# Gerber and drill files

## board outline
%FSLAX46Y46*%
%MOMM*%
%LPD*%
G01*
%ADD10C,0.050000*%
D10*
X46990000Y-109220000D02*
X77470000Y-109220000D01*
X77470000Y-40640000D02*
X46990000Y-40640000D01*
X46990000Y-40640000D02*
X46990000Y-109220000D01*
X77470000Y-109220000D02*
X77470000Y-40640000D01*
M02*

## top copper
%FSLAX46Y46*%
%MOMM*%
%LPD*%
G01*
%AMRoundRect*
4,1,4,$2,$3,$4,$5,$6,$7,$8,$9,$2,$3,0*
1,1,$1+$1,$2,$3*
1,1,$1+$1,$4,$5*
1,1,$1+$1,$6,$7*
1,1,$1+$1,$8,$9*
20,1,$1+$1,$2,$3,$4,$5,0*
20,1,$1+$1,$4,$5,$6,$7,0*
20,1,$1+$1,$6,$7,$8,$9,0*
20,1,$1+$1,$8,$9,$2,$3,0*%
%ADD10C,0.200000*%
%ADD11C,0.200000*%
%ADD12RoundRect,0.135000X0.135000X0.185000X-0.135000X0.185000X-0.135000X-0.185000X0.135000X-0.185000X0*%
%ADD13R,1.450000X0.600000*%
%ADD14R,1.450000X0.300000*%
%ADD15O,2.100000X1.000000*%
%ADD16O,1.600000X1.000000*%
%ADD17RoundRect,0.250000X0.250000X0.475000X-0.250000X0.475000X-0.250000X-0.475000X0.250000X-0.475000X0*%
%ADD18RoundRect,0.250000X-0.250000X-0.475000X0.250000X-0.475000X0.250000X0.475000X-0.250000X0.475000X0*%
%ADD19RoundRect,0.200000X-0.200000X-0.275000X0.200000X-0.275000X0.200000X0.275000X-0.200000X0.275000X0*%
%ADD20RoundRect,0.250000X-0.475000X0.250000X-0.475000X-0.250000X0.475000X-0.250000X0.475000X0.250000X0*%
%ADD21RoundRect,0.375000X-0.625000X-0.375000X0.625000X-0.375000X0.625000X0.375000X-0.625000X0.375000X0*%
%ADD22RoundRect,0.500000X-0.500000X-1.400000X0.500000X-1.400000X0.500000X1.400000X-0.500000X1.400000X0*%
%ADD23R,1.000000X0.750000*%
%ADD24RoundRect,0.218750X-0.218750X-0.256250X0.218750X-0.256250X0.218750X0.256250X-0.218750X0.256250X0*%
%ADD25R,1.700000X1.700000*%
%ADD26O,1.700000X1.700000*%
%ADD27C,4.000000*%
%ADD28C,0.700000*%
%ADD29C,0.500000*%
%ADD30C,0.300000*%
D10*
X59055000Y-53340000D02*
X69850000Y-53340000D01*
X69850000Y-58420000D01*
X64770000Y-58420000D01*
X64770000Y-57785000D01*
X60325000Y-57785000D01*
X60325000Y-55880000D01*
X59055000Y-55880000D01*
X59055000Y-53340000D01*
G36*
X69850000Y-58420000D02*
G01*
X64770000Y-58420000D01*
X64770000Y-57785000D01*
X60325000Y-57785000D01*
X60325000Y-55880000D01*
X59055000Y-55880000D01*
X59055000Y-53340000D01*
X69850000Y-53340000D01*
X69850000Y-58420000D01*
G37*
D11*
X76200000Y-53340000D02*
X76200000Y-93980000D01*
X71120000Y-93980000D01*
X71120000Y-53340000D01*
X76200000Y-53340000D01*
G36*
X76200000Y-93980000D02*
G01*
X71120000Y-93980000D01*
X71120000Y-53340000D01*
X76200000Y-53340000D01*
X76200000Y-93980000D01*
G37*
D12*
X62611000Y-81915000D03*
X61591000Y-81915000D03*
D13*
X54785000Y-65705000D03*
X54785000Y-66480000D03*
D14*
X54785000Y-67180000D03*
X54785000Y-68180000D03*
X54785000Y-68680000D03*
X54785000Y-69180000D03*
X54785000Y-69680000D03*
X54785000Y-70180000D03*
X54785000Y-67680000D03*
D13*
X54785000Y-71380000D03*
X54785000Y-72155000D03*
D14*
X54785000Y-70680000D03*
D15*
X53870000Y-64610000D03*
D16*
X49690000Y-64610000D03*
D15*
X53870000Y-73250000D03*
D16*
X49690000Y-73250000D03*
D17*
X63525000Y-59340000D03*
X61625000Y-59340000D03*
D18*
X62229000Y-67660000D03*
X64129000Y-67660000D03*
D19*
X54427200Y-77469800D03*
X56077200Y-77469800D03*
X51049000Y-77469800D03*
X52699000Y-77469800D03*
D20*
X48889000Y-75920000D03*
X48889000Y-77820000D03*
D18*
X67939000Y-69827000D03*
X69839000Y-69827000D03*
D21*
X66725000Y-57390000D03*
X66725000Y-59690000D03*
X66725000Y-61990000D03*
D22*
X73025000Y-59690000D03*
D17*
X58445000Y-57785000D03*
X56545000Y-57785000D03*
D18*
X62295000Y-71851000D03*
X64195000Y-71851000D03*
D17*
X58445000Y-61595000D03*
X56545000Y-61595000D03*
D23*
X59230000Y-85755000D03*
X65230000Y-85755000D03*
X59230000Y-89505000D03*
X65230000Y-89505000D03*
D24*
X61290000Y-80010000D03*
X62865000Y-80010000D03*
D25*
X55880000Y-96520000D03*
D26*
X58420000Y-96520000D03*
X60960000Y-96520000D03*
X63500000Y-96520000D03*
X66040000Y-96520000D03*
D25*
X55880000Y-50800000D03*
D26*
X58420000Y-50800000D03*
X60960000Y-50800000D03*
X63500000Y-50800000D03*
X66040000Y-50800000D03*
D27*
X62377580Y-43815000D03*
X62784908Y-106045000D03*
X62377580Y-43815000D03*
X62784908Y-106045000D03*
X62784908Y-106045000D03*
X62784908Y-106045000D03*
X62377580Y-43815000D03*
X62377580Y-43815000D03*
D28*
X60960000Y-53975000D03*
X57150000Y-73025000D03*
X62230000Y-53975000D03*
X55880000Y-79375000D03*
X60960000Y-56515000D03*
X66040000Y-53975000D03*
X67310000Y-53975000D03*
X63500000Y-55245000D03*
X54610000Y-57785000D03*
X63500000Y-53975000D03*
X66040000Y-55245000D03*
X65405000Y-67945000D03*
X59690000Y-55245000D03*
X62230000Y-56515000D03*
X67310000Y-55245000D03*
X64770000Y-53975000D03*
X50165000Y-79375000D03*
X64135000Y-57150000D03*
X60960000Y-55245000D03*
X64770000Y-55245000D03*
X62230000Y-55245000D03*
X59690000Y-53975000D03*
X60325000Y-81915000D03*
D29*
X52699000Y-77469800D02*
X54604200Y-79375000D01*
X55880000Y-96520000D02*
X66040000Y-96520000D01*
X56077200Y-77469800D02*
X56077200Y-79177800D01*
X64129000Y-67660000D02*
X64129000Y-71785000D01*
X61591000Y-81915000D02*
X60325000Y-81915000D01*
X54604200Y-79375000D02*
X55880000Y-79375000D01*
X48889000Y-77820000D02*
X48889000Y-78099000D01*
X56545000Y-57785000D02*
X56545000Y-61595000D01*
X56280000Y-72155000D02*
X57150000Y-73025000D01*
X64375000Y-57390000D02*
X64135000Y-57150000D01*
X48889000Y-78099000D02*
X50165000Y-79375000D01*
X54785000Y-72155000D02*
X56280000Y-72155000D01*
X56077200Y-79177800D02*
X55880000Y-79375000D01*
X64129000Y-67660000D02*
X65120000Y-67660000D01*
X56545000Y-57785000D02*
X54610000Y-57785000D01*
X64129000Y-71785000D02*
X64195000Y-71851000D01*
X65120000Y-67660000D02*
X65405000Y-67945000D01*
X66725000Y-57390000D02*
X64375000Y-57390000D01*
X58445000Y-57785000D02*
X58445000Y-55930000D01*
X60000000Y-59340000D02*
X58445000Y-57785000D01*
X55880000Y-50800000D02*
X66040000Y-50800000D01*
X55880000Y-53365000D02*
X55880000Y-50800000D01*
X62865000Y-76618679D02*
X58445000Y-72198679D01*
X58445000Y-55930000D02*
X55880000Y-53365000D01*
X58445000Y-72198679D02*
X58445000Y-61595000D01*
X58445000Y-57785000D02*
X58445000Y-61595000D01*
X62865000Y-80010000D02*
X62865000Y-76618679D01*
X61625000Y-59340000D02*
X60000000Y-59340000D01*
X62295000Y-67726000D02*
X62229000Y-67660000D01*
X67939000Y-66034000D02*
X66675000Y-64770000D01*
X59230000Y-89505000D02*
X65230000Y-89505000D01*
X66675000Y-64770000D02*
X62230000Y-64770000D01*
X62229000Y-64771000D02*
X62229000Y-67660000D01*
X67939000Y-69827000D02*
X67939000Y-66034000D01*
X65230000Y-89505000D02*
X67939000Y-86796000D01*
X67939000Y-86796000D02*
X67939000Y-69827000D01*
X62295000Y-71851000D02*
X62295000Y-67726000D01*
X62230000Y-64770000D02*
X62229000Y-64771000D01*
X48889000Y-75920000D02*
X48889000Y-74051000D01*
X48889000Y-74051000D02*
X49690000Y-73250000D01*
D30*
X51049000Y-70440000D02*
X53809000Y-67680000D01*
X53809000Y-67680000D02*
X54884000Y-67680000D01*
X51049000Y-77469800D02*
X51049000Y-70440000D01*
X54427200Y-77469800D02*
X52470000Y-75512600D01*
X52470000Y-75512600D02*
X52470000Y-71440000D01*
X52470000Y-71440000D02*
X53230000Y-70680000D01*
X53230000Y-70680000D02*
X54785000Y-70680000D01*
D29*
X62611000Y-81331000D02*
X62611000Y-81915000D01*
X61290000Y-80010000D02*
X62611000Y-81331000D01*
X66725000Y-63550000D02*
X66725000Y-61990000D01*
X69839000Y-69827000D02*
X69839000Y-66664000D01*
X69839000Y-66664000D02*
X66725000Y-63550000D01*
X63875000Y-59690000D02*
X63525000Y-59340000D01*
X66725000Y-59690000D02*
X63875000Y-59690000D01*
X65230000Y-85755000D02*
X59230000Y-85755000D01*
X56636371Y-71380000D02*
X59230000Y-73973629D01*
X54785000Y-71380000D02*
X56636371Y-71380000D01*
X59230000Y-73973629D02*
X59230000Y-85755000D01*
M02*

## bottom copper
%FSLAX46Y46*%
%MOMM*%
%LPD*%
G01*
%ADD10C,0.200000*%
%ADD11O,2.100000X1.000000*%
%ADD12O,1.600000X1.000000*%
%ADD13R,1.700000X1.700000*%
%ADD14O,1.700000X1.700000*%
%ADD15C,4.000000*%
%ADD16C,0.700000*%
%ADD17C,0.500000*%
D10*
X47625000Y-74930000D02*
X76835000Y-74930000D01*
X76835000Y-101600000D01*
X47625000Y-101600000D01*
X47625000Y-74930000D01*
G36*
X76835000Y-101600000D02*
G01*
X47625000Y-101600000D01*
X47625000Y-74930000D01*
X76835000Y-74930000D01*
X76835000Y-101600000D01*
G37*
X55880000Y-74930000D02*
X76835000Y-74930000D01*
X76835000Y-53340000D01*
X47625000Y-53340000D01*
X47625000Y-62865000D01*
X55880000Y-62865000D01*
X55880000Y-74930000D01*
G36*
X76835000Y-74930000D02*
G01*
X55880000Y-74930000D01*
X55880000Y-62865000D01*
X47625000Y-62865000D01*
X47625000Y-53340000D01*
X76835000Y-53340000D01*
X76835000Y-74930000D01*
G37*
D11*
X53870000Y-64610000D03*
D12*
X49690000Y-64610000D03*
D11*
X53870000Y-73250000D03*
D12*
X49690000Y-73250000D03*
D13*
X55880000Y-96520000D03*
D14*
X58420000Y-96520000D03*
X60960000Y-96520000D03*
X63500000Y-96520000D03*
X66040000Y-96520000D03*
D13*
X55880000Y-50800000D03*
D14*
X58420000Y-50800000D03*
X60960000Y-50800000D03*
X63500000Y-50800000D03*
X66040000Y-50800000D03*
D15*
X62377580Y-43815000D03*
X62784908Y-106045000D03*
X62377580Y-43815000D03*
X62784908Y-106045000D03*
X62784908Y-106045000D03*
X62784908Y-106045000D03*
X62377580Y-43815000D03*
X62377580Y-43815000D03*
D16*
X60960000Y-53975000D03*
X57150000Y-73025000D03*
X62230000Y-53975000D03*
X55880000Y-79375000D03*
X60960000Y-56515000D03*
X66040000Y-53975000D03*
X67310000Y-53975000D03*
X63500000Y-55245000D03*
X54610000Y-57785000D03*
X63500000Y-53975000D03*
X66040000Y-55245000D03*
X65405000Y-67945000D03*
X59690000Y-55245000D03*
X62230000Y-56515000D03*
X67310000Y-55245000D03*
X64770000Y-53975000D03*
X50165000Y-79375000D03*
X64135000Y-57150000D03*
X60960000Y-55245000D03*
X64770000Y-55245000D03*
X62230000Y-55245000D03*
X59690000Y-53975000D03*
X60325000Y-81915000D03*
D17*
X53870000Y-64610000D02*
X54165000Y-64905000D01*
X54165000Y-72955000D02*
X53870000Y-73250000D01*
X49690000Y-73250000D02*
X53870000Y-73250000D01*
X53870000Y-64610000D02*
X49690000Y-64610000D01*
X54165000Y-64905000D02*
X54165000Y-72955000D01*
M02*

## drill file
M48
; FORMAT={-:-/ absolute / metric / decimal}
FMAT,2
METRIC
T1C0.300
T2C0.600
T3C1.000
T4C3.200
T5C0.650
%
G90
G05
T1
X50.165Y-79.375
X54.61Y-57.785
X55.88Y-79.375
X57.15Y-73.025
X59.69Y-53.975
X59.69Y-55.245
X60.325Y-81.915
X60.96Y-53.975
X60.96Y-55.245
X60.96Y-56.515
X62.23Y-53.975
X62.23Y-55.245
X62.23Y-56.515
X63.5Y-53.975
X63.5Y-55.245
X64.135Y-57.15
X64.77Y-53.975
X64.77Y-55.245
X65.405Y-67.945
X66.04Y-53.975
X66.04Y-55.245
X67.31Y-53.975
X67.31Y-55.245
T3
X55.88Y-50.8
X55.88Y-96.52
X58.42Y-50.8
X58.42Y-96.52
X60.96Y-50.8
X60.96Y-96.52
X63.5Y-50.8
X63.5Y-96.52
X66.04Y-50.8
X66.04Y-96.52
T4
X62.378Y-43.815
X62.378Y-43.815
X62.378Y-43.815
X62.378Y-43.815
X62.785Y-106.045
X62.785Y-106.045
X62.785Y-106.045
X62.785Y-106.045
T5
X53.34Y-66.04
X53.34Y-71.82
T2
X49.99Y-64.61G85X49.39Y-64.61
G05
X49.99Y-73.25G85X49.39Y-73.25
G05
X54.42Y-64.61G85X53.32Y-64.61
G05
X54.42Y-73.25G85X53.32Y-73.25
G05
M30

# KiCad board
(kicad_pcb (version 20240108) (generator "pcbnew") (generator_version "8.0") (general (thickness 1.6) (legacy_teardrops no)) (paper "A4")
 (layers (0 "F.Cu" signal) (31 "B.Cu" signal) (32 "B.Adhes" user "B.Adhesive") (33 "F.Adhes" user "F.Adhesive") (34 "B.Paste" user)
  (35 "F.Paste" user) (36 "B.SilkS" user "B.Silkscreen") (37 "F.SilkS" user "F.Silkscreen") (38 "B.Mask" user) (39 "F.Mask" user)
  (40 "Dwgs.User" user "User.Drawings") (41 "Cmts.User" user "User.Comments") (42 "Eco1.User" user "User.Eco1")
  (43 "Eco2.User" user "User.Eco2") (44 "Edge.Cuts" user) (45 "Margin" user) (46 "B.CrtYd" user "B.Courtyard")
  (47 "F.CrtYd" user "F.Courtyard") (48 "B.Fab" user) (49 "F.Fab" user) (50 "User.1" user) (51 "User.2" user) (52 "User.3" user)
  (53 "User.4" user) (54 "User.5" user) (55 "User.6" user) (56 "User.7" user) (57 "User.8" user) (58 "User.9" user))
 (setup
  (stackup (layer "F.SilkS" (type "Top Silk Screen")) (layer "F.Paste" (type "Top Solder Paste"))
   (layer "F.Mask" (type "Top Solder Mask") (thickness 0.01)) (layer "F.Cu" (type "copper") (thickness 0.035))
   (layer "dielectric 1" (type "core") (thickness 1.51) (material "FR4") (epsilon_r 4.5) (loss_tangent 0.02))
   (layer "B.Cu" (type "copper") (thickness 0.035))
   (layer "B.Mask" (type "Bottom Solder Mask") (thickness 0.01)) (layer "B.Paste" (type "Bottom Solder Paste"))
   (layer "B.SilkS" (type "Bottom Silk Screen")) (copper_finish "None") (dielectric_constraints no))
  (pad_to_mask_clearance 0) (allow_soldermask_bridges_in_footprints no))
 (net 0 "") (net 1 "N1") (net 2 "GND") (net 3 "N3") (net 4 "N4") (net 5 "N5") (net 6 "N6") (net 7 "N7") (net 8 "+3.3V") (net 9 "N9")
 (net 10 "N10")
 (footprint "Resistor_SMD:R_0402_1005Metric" (layer "F.Cu") (at 62.101 81.915 180)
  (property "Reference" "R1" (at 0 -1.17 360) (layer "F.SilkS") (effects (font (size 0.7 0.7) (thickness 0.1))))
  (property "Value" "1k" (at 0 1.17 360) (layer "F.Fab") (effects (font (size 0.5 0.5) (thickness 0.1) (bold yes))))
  (pad "1" smd roundrect (at -0.51 0 180) (size 0.54 0.64) (layers "F.Cu" "F.Paste" "F.Mask") (roundrect_rratio 0.25) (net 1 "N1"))
  (pad "2" smd roundrect (at 0.51 0 180) (size 0.54 0.64) (layers "F.Cu" "F.Paste" "F.Mask") (roundrect_rratio 0.25) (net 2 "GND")))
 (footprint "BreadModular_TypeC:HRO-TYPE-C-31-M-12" (layer "F.Cu") (at 47.09 68.93 -90)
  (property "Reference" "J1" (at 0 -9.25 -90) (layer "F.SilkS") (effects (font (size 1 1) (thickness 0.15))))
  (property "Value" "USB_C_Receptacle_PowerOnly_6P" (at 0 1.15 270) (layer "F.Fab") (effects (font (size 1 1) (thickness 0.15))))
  (pad "" np_thru_hole circle (at -2.89 -6.25 270) (size 0.65 0.65) (drill 0.65) (layers "*.Cu" "*.Mask"))
  (pad "" np_thru_hole circle (at 2.89 -6.25 270) (size 0.65 0.65) (drill 0.65) (layers "*.Cu" "*.Mask"))
  (pad "1" smd rect (at -3.225 -7.695 270) (size 0.6 1.45) (layers "F.Cu" "F.Paste" "F.Mask"))
  (pad "2" smd rect (at -2.45 -7.695 270) (size 0.6 1.45) (layers "F.Cu" "F.Paste" "F.Mask"))
  (pad "3" smd rect (at -1.75 -7.695 270) (size 0.3 1.45) (layers "F.Cu" "F.Paste" "F.Mask"))
  (pad "5" smd rect (at -0.75 -7.695 270) (size 0.3 1.45) (layers "F.Cu" "F.Paste" "F.Mask"))
  (pad "6" smd rect (at -0.25 -7.695 270) (size 0.3 1.45) (layers "F.Cu" "F.Paste" "F.Mask"))
  (pad "7" smd rect (at 0.25 -7.695 270) (size 0.3 1.45) (layers "F.Cu" "F.Paste" "F.Mask"))
  (pad "8" smd rect (at 0.75 -7.695 270) (size 0.3 1.45) (layers "F.Cu" "F.Paste" "F.Mask"))
  (pad "9" smd rect (at 1.25 -7.695 270) (size 0.3 1.45) (layers "F.Cu" "F.Paste" "F.Mask"))
  (pad "A5" smd rect (at -1.25 -7.695 270) (size 0.3 1.45) (layers "F.Cu" "F.Paste" "F.Mask") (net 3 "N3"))
  (pad "A9" smd rect (at 2.45 -7.695 270) (size 0.6 1.45) (layers "F.Cu" "F.Paste" "F.Mask") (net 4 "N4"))
  (pad "A12" smd rect (at 3.225 -7.695 270) (size 0.6 1.45) (layers "F.Cu" "F.Paste" "F.Mask") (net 2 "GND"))
  (pad "B5" smd rect (at 1.75 -7.695 270) (size 0.3 1.45) (layers "F.Cu" "F.Paste" "F.Mask") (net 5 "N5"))
  (pad "S1" thru_hole oval (at -4.32 -6.78 270) (size 1 2.1) (drill oval 0.6 1.7) (layers "*.Cu" "F.Paste" "B.Mask")
   (remove_unused_layers no) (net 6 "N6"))
  (pad "S1" thru_hole oval (at -4.32 -2.6 270) (size 1 1.6) (drill oval 0.6 1.2) (layers "*.Cu" "F.Paste" "B.Mask" "Eco2.User")
   (remove_unused_layers no) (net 6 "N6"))
  (pad "S1" thru_hole oval (at 4.32 -6.78 270) (size 1 2.1) (drill oval 0.6 1.7) (layers "*.Cu" "F.Paste" "B.Mask")
   (remove_unused_layers no) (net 6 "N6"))
  (pad "S1" thru_hole oval (at 4.32 -2.6 270) (size 1 1.6) (drill oval 0.6 1.2) (layers "*.Cu" "F.Paste" "B.Mask") (remove_unused_layers no)
   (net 6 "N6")))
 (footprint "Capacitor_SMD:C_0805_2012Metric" (layer "F.Cu") (at 62.575 59.34 180)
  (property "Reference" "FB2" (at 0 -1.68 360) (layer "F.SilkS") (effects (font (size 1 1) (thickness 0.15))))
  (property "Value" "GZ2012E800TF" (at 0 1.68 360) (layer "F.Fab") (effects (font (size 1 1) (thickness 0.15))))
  (pad "1" smd roundrect (at -0.95 0 180) (size 1 1.45) (layers "F.Cu" "F.Paste" "F.Mask") (roundrect_rratio 0.25) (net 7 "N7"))
  (pad "2" smd roundrect (at 0.95 0 180) (size 1 1.45) (layers "F.Cu" "F.Paste" "F.Mask") (roundrect_rratio 0.25) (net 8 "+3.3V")))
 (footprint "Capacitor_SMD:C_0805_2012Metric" (layer "F.Cu") (at 63.179 67.66)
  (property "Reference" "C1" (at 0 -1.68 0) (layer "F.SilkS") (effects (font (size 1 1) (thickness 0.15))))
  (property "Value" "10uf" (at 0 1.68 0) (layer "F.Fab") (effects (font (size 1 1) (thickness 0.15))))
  (pad "1" smd roundrect (at -0.95 0) (size 1 1.45) (layers "F.Cu" "F.Paste" "F.Mask") (roundrect_rratio 0.25) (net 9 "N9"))
  (pad "2" smd roundrect (at 0.95 0) (size 1 1.45) (layers "F.Cu" "F.Paste" "F.Mask") (roundrect_rratio 0.25) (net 2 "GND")))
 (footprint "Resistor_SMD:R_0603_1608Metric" (layer "F.Cu") (at 55.2522 77.4698)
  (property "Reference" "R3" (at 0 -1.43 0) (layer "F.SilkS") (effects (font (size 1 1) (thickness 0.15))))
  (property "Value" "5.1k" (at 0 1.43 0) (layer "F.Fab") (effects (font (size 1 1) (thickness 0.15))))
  (pad "1" smd roundrect (at -0.825 0) (size 0.8 0.95) (layers "F.Cu" "F.Paste" "F.Mask") (roundrect_rratio 0.25) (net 5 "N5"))
  (pad "2" smd roundrect (at 0.825 0) (size 0.8 0.95) (layers "F.Cu" "F.Paste" "F.Mask") (roundrect_rratio 0.25) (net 2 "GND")))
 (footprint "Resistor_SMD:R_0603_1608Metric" (layer "F.Cu") (at 51.874 77.4698)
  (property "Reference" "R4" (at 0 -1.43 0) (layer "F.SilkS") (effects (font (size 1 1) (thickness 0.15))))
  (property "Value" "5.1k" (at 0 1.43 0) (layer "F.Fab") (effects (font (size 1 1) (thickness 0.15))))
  (pad "1" smd roundrect (at -0.825 0) (size 0.8 0.95) (layers "F.Cu" "F.Paste" "F.Mask") (roundrect_rratio 0.25) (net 3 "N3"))
  (pad "2" smd roundrect (at 0.825 0) (size 0.8 0.95) (layers "F.Cu" "F.Paste" "F.Mask") (roundrect_rratio 0.25) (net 2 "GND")))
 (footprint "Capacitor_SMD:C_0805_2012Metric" (layer "F.Cu") (at 48.889 76.87 -90)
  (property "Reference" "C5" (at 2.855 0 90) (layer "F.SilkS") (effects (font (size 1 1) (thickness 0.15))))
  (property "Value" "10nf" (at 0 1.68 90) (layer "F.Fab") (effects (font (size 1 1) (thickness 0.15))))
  (pad "1" smd roundrect (at -0.95 0 270) (size 1 1.45) (layers "F.Cu" "F.Paste" "F.Mask") (roundrect_rratio 0.25) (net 6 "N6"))
  (pad "2" smd roundrect (at 0.95 0 270) (size 1 1.45) (layers "F.Cu" "F.Paste" "F.Mask") (roundrect_rratio 0.25) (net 2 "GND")))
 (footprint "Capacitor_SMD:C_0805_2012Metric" (layer "F.Cu") (at 68.889 69.827)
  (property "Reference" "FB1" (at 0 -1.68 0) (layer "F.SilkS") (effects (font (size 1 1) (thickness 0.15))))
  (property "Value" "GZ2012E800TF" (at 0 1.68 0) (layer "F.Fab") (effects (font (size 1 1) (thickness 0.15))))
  (pad "1" smd roundrect (at -0.95 0) (size 1 1.45) (layers "F.Cu" "F.Paste" "F.Mask") (roundrect_rratio 0.25) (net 9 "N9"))
  (pad "2" smd roundrect (at 0.95 0) (size 1 1.45) (layers "F.Cu" "F.Paste" "F.Mask") (roundrect_rratio 0.25) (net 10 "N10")))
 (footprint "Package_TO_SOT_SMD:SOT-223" (layer "F.Cu") (at 69.875 59.69)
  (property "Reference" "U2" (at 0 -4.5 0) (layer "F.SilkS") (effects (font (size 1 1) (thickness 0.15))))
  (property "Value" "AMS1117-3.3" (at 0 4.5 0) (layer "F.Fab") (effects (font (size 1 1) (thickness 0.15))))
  (pad "1" smd roundrect (at -3.15 -2.3) (size 2 1.5) (layers "F.Cu" "F.Paste" "F.Mask") (roundrect_rratio 0.25) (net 2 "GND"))
  (pad "2" smd roundrect (at -3.15 0) (size 2 1.5) (layers "F.Cu" "F.Paste" "F.Mask") (roundrect_rratio 0.25) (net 7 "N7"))
  (pad "3" smd roundrect (at -3.15 2.3) (size 2 1.5) (layers "F.Cu" "F.Paste" "F.Mask") (roundrect_rratio 0.25) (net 10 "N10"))
  (pad "4" smd roundrect (at 3.15 0) (size 2 3.8) (layers "F.Cu" "F.Paste" "F.Mask") (roundrect_rratio 0.25)))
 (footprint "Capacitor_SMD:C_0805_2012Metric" (layer "F.Cu") (at 57.495 57.785 180)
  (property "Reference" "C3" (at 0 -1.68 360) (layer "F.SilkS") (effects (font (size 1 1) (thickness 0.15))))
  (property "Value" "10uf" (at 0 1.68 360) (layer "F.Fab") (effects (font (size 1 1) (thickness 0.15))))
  (pad "1" smd roundrect (at -0.95 0 180) (size 1 1.45) (layers "F.Cu" "F.Paste" "F.Mask") (roundrect_rratio 0.25) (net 8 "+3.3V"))
  (pad "2" smd roundrect (at 0.95 0 180) (size 1 1.45) (layers "F.Cu" "F.Paste" "F.Mask") (roundrect_rratio 0.25) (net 2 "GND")))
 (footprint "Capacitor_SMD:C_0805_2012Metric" (layer "F.Cu") (at 63.245 71.851)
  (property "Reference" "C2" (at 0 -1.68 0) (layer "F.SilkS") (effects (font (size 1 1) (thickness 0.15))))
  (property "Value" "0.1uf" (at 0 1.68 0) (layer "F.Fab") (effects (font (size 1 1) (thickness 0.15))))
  (pad "1" smd roundrect (at -0.95 0) (size 1 1.45) (layers "F.Cu" "F.Paste" "F.Mask") (roundrect_rratio 0.25) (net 9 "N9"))
  (pad "2" smd roundrect (at 0.95 0) (size 1 1.45) (layers "F.Cu" "F.Paste" "F.Mask") (roundrect_rratio 0.25) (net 2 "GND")))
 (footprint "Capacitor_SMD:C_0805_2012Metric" (layer "F.Cu") (at 57.495 61.595 180)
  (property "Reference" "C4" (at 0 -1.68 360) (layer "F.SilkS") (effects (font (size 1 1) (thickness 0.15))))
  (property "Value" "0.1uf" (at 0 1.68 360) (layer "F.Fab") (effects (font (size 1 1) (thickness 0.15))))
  (pad "1" smd roundrect (at -0.95 0 180) (size 1 1.45) (layers "F.Cu" "F.Paste" "F.Mask") (roundrect_rratio 0.25) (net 8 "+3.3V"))
  (pad "2" smd roundrect (at 0.95 0 180) (size 1 1.45) (layers "F.Cu" "F.Paste" "F.Mask") (roundrect_rratio 0.25) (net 2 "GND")))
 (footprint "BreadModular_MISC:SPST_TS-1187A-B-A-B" (layer "F.Cu") (at 62.23 87.63)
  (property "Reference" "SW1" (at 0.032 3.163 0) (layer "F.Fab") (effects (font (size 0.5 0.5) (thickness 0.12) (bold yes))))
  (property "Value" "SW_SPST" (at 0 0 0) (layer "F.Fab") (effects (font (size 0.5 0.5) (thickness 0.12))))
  (pad "1" smd rect (at -3 -1.875) (size 1 0.75) (layers "F.Cu" "F.Paste" "F.Mask") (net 4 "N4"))
  (pad "1" smd rect (at 3 -1.875) (size 1 0.75) (layers "F.Cu" "F.Paste" "F.Mask") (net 4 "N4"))
  (pad "2" smd rect (at -3 1.875) (size 1 0.75) (layers "F.Cu" "F.Paste" "F.Mask") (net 9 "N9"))
  (pad "2" smd rect (at 3 1.875) (size 1 0.75) (layers "F.Cu" "F.Paste" "F.Mask") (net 9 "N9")))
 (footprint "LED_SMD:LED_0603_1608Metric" (layer "F.Cu") (at 62.0775 80.01)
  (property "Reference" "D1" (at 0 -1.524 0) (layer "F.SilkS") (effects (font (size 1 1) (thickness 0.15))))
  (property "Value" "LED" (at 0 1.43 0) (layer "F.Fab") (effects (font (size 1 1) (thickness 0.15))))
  (pad "1" smd roundrect (at -0.7875 0) (size 0.875 0.95) (layers "F.Cu" "F.Paste" "F.Mask") (roundrect_rratio 0.25) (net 1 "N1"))
  (pad "2" smd roundrect (at 0.7875 0) (size 0.875 0.95) (layers "F.Cu" "F.Paste" "F.Mask") (roundrect_rratio 0.25) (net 8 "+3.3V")))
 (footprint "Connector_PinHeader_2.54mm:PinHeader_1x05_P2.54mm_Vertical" (layer "B.Cu") (at 55.88 96.52 -90)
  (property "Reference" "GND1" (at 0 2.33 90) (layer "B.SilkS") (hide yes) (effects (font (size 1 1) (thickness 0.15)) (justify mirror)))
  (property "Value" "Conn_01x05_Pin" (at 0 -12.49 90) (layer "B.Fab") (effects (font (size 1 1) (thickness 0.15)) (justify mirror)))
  (pad "1" thru_hole rect (at 0 0 270) (size 1.7 1.7) (drill 1) (layers "*.Cu" "*.Mask") (remove_unused_layers no) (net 2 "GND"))
  (pad "2" thru_hole oval (at 0 -2.54 270) (size 1.7 1.7) (drill 1) (layers "*.Cu" "*.Mask") (remove_unused_layers no) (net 2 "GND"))
  (pad "3" thru_hole oval (at 0 -5.08 270) (size 1.7 1.7) (drill 1) (layers "*.Cu" "*.Mask") (remove_unused_layers no) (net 2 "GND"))
  (pad "4" thru_hole oval (at 0 -7.62 270) (size 1.7 1.7) (drill 1) (layers "*.Cu" "*.Mask") (remove_unused_layers no) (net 2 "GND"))
  (pad "5" thru_hole oval (at 0 -10.16 270) (size 1.7 1.7) (drill 1) (layers "*.Cu" "*.Mask") (remove_unused_layers no) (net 2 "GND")))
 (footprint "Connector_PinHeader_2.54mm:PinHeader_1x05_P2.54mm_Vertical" (layer "B.Cu") (at 55.88 50.8 -90)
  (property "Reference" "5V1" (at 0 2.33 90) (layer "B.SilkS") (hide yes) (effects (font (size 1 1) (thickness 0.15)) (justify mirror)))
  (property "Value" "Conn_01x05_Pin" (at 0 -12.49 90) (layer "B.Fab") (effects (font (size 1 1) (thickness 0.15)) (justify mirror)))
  (pad "1" thru_hole rect (at 0 0 270) (size 1.7 1.7) (drill 1) (layers "*.Cu" "*.Mask") (remove_unused_layers no) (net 8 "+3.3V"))
  (pad "2" thru_hole oval (at 0 -2.54 270) (size 1.7 1.7) (drill 1) (layers "*.Cu" "*.Mask") (remove_unused_layers no) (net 8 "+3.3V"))
  (pad "3" thru_hole oval (at 0 -5.08 270) (size 1.7 1.7) (drill 1) (layers "*.Cu" "*.Mask") (remove_unused_layers no) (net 8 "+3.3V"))
  (pad "4" thru_hole oval (at 0 -7.62 270) (size 1.7 1.7) (drill 1) (layers "*.Cu" "*.Mask") (remove_unused_layers no) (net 8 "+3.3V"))
  (pad "5" thru_hole oval (at 0 -10.16 270) (size 1.7 1.7) (drill 1) (layers "*.Cu" "*.Mask") (remove_unused_layers no) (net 8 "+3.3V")))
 (gr_poly
  (pts (xy 59.055 53.34) (xy 69.85 53.34) (xy 69.85 58.42) (xy 64.77 58.42) (xy 64.77 57.785) (xy 60.325 57.785) (xy 60.325 55.88)
   (xy 59.055 55.88))
  (stroke (width 0.2) (type solid)) (fill solid) (layer "F.Cu") (net 2))
 (gr_poly
  (pts (xy 76.2 53.34) (xy 76.2 93.98) (xy 71.12 93.98) (xy 71.12 53.34)) (stroke (width 0.2) (type solid)) (fill solid) (layer "F.Cu"))
 (gr_poly
  (pts (xy 47.625 74.93) (xy 76.835 74.93) (xy 76.835 101.6) (xy 47.625 101.6)) (stroke (width 0.2) (type solid)) (fill solid)
  (layer "B.Cu") (net 2))
 (gr_poly
  (pts (xy 55.88 74.93) (xy 76.835 74.93) (xy 76.835 53.34) (xy 47.625 53.34) (xy 47.625 62.865) (xy 55.88 62.865))
  (stroke (width 0.2) (type solid)) (fill solid) (layer "B.Cu") (net 2))
 (gr_line (start 46.99 109.22) (end 77.47 109.22) (stroke (width 0.05) (type default)) (layer "Edge.Cuts"))
 (gr_line (start 77.47 40.64) (end 46.99 40.64) (stroke (width 0.05) (type default)) (layer "Edge.Cuts"))
 (gr_line (start 46.99 40.64) (end 46.99 109.22) (stroke (width 0.05) (type default)) (layer "Edge.Cuts"))
 (gr_line (start 77.47 109.22) (end 77.47 40.64) (stroke (width 0.05) (type default)) (layer "Edge.Cuts"))
 (via (at 62.37758 43.815) (size 4) (drill 3.2) (layers "F.Cu" "B.Cu") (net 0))
 (via (at 62.784908 106.045) (size 4) (drill 3.2) (layers "F.Cu" "B.Cu") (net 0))
 (via (at 62.37758 43.815) (size 4) (drill 3.2) (layers "F.Cu" "B.Cu") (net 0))
 (via (at 62.784908 106.045) (size 4) (drill 3.2) (layers "F.Cu" "B.Cu") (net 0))
 (via (at 62.784908 106.045) (size 4) (drill 3.2) (layers "F.Cu" "B.Cu") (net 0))
 (via (at 62.784908 106.045) (size 4) (drill 3.2) (layers "F.Cu" "B.Cu") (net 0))
 (via (at 62.37758 43.815) (size 4) (drill 3.2) (layers "F.Cu" "B.Cu") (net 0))
 (via (at 62.37758 43.815) (size 4) (drill 3.2) (layers "F.Cu" "B.Cu") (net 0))
 (segment (start 52.699 77.4698) (end 54.6042 79.375) (width 0.5) (layer "F.Cu") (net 2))
 (segment (start 55.88 96.52) (end 66.04 96.52) (width 0.5) (layer "F.Cu") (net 2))
 (segment (start 56.0772 77.4698) (end 56.0772 79.1778) (width 0.5) (layer "F.Cu") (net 2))
 (segment (start 64.129 67.66) (end 64.129 71.785) (width 0.5) (layer "F.Cu") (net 2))
 (segment (start 61.591 81.915) (end 60.325 81.915) (width 0.5) (layer "F.Cu") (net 2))
 (segment (start 54.6042 79.375) (end 55.88 79.375) (width 0.5) (layer "F.Cu") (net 2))
 (segment (start 48.889 77.82) (end 48.889 78.099) (width 0.5) (layer "F.Cu") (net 2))
 (segment (start 56.545 57.785) (end 56.545 61.595) (width 0.5) (layer "F.Cu") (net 2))
 (segment (start 56.28 72.155) (end 57.15 73.025) (width 0.5) (layer "F.Cu") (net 2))
 (segment (start 64.375 57.39) (end 64.135 57.15) (width 0.5) (layer "F.Cu") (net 2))
 (segment (start 48.889 78.099) (end 50.165 79.375) (width 0.5) (layer "F.Cu") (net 2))
 (segment (start 54.785 72.155) (end 56.28 72.155) (width 0.5) (layer "F.Cu") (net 2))
 (segment (start 56.0772 79.1778) (end 55.88 79.375) (width 0.5) (layer "F.Cu") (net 2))
 (segment (start 64.129 67.66) (end 65.12 67.66) (width 0.5) (layer "F.Cu") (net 2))
 (segment (start 56.545 57.785) (end 54.61 57.785) (width 0.5) (layer "F.Cu") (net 2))
 (segment (start 64.129 71.785) (end 64.195 71.851) (width 0.5) (layer "F.Cu") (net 2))
 (segment (start 65.12 67.66) (end 65.405 67.945) (width 0.5) (layer "F.Cu") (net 2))
 (segment (start 66.725 57.39) (end 64.375 57.39) (width 0.5) (layer "F.Cu") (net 2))
 (via (at 60.96 53.975) (size 0.7) (drill 0.3) (layers "F.Cu" "B.Cu") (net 2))
 (via (at 57.15 73.025) (size 0.7) (drill 0.3) (layers "F.Cu" "B.Cu") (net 2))
 (via (at 62.23 53.975) (size 0.7) (drill 0.3) (layers "F.Cu" "B.Cu") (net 2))
 (via (at 55.88 79.375) (size 0.7) (drill 0.3) (layers "F.Cu" "B.Cu") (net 2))
 (via (at 60.96 56.515) (size 0.7) (drill 0.3) (layers "F.Cu" "B.Cu") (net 2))
 (via (at 66.04 53.975) (size 0.7) (drill 0.3) (layers "F.Cu" "B.Cu") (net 2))
 (via (at 67.31 53.975) (size 0.7) (drill 0.3) (layers "F.Cu" "B.Cu") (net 2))
 (via (at 63.5 55.245) (size 0.7) (drill 0.3) (layers "F.Cu" "B.Cu") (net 2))
 (via (at 54.61 57.785) (size 0.7) (drill 0.3) (layers "F.Cu" "B.Cu") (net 2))
 (via (at 63.5 53.975) (size 0.7) (drill 0.3) (layers "F.Cu" "B.Cu") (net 2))
 (via (at 66.04 55.245) (size 0.7) (drill 0.3) (layers "F.Cu" "B.Cu") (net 2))
 (via (at 65.405 67.945) (size 0.7) (drill 0.3) (layers "F.Cu" "B.Cu") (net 2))
 (via (at 59.69 55.245) (size 0.7) (drill 0.3) (layers "F.Cu" "B.Cu") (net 2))
 (via (at 62.23 56.515) (size 0.7) (drill 0.3) (layers "F.Cu" "B.Cu") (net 2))
 (via (at 67.31 55.245) (size 0.7) (drill 0.3) (layers "F.Cu" "B.Cu") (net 2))
 (via (at 64.77 53.975) (size 0.7) (drill 0.3) (layers "F.Cu" "B.Cu") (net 2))
 (via (at 50.165 79.375) (size 0.7) (drill 0.3) (layers "F.Cu" "B.Cu") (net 2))
 (via (at 64.135 57.15) (size 0.7) (drill 0.3) (layers "F.Cu" "B.Cu") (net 2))
 (via (at 60.96 55.245) (size 0.7) (drill 0.3) (layers "F.Cu" "B.Cu") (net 2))
 (via (at 64.77 55.245) (size 0.7) (drill 0.3) (layers "F.Cu" "B.Cu") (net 2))
 (via (at 62.23 55.245) (size 0.7) (drill 0.3) (layers "F.Cu" "B.Cu") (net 2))
 (via (at 59.69 53.975) (size 0.7) (drill 0.3) (layers "F.Cu" "B.Cu") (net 2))
 (via (at 60.325 81.915) (size 0.7) (drill 0.3) (layers "F.Cu" "B.Cu") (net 2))
 (segment (start 58.445 57.785) (end 58.445 55.93) (width 0.5) (layer "F.Cu") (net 8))
 (segment (start 60 59.34) (end 58.445 57.785) (width 0.5) (layer "F.Cu") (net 8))
 (segment (start 55.88 50.8) (end 66.04 50.8) (width 0.5) (layer "F.Cu") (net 8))
 (segment (start 55.88 53.365) (end 55.88 50.8) (width 0.5) (layer "F.Cu") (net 8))
 (segment (start 62.865 76.618679) (end 58.445 72.198679) (width 0.5) (layer "F.Cu") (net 8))
 (segment (start 58.445 55.93) (end 55.88 53.365) (width 0.5) (layer "F.Cu") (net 8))
 (segment (start 58.445 72.198679) (end 58.445 61.595) (width 0.5) (layer "F.Cu") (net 8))
 (segment (start 58.445 57.785) (end 58.445 61.595) (width 0.5) (layer "F.Cu") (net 8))
 (segment (start 62.865 80.01) (end 62.865 76.618679) (width 0.5) (layer "F.Cu") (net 8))
 (segment (start 61.625 59.34) (end 60 59.34) (width 0.5) (layer "F.Cu") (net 8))
 (segment (start 62.295 67.726) (end 62.229 67.66) (width 0.5) (layer "F.Cu") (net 9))
 (segment (start 67.939 66.034) (end 66.675 64.77) (width 0.5) (layer "F.Cu") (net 9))
 (segment (start 59.23 89.505) (end 65.23 89.505) (width 0.5) (layer "F.Cu") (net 9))
 (segment (start 66.675 64.77) (end 62.23 64.77) (width 0.5) (layer "F.Cu") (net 9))
 (segment (start 62.229 64.771) (end 62.229 67.66) (width 0.5) (layer "F.Cu") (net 9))
 (segment (start 67.939 69.827) (end 67.939 66.034) (width 0.5) (layer "F.Cu") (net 9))
 (segment (start 65.23 89.505) (end 67.939 86.796) (width 0.5) (layer "F.Cu") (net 9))
 (segment (start 67.939 86.796) (end 67.939 69.827) (width 0.5) (layer "F.Cu") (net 9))
 (segment (start 62.295 71.851) (end 62.295 67.726) (width 0.5) (layer "F.Cu") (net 9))
 (segment (start 62.23 64.77) (end 62.229 64.771) (width 0.5) (layer "F.Cu") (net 9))
 (segment (start 48.889 75.92) (end 48.889 74.051) (width 0.5) (layer "F.Cu") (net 6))
 (segment (start 48.889 74.051) (end 49.69 73.25) (width 0.5) (layer "F.Cu") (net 6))
 (segment (start 53.87 64.61) (end 54.165 64.905) (width 0.5) (layer "B.Cu") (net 6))
 (segment (start 54.165 72.955) (end 53.87 73.25) (width 0.5) (layer "B.Cu") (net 6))
 (segment (start 49.69 73.25) (end 53.87 73.25) (width 0.5) (layer "B.Cu") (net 6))
 (segment (start 53.87 64.61) (end 49.69 64.61) (width 0.5) (layer "B.Cu") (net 6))
 (segment (start 54.165 64.905) (end 54.165 72.955) (width 0.5) (layer "B.Cu") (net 6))
 (segment (start 51.049 70.44) (end 53.809 67.68) (width 0.3) (layer "F.Cu") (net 3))
 (segment (start 53.809 67.68) (end 54.884 67.68) (width 0.3) (layer "F.Cu") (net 3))
 (segment (start 51.049 77.4698) (end 51.049 70.44) (width 0.3) (layer "F.Cu") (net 3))
 (segment (start 54.4272 77.4698) (end 52.47 75.5126) (width 0.3) (layer "F.Cu") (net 5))
 (segment (start 52.47 75.5126) (end 52.47 71.44) (width 0.3) (layer "F.Cu") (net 5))
 (segment (start 52.47 71.44) (end 53.23 70.68) (width 0.3) (layer "F.Cu") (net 5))
 (segment (start 53.23 70.68) (end 54.785 70.68) (width 0.3) (layer "F.Cu") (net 5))
 (segment (start 62.611 81.331) (end 62.611 81.915) (width 0.5) (layer "F.Cu") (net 1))
 (segment (start 61.29 80.01) (end 62.611 81.331) (width 0.5) (layer "F.Cu") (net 1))
 (segment (start 66.725 63.55) (end 66.725 61.99) (width 0.5) (layer "F.Cu") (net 10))
 (segment (start 69.839 69.827) (end 69.839 66.664) (width 0.5) (layer "F.Cu") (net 10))
 (segment (start 69.839 66.664) (end 66.725 63.55) (width 0.5) (layer "F.Cu") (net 10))
 (segment (start 63.875 59.69) (end 63.525 59.34) (width 0.5) (layer "F.Cu") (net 7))
 (segment (start 66.725 59.69) (end 63.875 59.69) (width 0.5) (layer "F.Cu") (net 7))
 (segment (start 65.23 85.755) (end 59.23 85.755) (width 0.5) (layer "F.Cu") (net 4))
 (segment (start 56.636371 71.38) (end 59.23 73.973629) (width 0.5) (layer "F.Cu") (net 4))
 (segment (start 54.785 71.38) (end 56.636371 71.38) (width 0.5) (layer "F.Cu") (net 4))
 (segment (start 59.23 73.973629) (end 59.23 85.755) (width 0.5) (layer "F.Cu") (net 4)))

